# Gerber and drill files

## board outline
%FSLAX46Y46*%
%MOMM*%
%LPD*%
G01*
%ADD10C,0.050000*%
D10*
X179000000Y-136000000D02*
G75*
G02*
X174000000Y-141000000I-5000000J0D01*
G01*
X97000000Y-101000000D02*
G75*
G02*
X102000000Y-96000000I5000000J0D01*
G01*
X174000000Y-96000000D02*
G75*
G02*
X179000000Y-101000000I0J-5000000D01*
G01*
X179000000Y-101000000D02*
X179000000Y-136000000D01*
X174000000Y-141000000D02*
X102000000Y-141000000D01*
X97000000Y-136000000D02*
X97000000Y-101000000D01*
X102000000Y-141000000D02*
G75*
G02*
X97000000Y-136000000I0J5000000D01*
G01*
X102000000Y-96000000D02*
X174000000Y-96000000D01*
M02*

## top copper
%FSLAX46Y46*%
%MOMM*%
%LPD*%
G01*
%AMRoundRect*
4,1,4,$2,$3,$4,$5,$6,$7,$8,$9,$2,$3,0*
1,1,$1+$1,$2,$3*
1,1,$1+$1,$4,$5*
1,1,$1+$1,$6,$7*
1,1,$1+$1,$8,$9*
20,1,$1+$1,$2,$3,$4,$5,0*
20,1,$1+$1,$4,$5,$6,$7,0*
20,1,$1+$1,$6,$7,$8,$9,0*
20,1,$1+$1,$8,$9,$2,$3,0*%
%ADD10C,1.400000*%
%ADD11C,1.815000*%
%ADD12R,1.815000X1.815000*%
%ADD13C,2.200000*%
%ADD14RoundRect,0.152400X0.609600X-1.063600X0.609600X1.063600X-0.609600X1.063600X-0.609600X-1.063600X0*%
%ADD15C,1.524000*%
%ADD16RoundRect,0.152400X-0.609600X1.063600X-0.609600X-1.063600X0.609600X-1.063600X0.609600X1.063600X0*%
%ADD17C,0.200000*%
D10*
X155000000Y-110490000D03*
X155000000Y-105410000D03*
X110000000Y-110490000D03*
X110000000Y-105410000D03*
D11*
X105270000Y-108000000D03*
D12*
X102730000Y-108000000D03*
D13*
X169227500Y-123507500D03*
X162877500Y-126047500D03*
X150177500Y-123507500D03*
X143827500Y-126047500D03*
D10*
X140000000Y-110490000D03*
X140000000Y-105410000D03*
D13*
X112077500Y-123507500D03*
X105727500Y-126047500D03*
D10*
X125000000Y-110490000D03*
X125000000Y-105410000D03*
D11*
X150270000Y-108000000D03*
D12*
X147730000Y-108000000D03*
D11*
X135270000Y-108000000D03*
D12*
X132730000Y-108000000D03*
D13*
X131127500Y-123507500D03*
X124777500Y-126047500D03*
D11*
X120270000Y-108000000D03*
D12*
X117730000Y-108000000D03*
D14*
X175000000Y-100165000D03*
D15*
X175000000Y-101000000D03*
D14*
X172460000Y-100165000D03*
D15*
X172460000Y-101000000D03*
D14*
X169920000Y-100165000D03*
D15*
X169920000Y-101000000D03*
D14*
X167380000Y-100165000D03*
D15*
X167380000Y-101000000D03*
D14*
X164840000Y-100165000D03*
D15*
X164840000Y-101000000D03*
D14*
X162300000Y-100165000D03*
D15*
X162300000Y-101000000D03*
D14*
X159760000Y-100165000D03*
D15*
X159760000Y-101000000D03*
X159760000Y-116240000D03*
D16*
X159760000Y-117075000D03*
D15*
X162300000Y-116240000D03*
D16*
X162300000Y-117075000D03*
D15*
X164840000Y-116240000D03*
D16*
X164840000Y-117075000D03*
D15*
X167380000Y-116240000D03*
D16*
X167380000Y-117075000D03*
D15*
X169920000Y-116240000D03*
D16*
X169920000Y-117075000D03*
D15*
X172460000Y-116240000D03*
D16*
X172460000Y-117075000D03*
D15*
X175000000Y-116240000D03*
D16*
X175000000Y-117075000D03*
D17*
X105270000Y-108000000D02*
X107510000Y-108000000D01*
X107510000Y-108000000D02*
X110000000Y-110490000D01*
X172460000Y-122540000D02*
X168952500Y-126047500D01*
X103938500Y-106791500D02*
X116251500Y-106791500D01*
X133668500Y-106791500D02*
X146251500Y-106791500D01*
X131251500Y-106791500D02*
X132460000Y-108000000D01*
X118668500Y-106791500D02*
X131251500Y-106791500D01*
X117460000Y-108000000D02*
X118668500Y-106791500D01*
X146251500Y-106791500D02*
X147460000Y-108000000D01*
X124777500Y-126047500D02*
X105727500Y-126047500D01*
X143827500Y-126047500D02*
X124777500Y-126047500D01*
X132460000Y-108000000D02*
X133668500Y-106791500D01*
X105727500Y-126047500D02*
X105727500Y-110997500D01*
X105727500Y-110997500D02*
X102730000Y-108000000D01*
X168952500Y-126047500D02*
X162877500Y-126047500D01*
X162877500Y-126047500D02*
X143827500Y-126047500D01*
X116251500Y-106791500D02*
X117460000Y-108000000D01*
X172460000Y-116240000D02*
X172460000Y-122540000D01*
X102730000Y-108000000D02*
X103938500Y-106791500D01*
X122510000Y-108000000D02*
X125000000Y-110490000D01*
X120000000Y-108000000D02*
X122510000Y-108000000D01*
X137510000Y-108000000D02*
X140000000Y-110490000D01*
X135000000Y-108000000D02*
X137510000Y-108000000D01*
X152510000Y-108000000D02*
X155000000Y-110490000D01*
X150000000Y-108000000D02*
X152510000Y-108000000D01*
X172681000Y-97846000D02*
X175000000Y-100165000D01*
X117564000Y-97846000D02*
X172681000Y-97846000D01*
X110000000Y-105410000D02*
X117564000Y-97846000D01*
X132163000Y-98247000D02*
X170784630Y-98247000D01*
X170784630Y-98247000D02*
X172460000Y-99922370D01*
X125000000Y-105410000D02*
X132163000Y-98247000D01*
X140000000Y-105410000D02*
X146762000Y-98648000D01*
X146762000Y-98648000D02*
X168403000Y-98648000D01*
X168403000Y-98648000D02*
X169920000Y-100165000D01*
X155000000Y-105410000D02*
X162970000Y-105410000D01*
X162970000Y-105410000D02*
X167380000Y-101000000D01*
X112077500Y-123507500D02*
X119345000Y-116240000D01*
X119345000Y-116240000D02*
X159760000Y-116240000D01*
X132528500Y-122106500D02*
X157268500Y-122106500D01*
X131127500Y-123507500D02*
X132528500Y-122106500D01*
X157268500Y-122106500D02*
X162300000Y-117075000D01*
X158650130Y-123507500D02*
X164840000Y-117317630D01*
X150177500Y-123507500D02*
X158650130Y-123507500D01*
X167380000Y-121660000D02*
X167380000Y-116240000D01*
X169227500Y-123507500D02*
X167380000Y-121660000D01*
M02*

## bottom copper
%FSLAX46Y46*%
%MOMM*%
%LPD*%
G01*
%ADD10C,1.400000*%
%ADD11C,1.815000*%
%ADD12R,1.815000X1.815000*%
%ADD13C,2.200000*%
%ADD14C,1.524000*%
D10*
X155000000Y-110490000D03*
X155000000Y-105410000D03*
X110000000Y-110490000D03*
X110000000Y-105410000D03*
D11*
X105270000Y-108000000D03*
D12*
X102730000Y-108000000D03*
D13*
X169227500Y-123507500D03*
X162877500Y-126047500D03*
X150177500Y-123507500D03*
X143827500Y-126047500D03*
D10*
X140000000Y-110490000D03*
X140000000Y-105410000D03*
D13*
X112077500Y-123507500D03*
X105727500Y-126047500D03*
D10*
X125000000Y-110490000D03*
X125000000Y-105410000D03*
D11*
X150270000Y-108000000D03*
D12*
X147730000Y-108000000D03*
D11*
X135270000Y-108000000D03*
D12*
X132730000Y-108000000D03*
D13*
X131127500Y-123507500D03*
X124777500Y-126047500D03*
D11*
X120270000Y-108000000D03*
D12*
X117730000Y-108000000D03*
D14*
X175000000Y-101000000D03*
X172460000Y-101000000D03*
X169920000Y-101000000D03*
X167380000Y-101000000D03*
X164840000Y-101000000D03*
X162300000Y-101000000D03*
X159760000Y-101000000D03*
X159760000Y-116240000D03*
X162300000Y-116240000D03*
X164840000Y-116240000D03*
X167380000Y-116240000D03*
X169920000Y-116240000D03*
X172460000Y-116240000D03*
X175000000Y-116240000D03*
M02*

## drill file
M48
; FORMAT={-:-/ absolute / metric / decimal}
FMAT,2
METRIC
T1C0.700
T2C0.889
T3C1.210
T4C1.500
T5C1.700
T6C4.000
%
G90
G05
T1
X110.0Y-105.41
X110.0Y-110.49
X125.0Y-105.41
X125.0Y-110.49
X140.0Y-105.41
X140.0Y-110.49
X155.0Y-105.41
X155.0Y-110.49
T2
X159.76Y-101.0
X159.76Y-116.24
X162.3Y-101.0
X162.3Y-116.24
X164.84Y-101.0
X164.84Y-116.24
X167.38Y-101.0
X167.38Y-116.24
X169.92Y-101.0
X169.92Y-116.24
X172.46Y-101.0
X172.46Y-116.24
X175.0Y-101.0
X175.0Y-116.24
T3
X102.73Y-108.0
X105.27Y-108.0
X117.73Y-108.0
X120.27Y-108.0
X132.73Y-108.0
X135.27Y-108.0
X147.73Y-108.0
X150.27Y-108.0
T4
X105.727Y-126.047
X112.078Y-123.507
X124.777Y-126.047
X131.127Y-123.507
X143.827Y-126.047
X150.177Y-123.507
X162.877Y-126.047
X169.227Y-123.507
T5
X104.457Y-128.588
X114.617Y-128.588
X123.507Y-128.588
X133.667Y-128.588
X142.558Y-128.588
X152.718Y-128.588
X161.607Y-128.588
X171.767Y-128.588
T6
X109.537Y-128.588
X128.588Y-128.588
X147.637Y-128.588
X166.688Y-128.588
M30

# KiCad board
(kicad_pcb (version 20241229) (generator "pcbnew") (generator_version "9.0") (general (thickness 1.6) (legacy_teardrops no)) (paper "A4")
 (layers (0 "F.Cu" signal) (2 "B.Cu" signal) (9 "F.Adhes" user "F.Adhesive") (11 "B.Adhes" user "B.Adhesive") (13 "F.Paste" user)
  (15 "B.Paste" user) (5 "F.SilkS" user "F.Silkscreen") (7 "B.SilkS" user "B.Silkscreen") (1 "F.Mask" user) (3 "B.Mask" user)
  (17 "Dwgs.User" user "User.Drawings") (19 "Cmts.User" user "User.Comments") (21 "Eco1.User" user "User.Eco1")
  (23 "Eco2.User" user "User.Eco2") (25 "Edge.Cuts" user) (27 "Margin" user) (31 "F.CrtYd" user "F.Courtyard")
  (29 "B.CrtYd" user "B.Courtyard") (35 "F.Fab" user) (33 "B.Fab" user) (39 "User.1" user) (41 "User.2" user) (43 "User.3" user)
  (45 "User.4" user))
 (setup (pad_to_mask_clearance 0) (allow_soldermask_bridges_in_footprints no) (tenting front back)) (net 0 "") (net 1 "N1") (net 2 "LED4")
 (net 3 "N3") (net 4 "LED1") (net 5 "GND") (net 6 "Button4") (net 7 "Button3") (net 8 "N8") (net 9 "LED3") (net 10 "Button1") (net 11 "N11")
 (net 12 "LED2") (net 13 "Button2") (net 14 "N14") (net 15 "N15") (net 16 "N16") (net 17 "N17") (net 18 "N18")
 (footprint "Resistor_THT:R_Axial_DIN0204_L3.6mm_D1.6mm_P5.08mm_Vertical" (layer "F.Cu") (at 155 110.49 90)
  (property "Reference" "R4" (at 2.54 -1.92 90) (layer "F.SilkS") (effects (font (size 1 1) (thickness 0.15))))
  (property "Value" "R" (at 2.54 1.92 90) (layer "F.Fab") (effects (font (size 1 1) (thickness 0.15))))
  (pad "1" thru_hole circle (at 0 0 90) (size 1.4 1.4) (drill 0.7) (layers "*.Cu" "*.Mask") (remove_unused_layers no) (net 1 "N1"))
  (pad "2" thru_hole circle (at 5.08 0 90) (size 1.4 1.4) (drill 0.7) (layers "*.Cu" "*.Mask") (remove_unused_layers no) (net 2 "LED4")))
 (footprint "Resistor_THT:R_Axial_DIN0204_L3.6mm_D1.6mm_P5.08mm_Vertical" (layer "F.Cu") (at 110 110.49 90)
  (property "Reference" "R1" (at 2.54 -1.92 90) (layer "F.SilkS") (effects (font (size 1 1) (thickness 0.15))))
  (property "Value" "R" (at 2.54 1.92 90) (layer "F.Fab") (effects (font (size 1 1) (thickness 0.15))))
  (pad "1" thru_hole circle (at 0 0 90) (size 1.4 1.4) (drill 0.7) (layers "*.Cu" "*.Mask") (remove_unused_layers no) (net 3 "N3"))
  (pad "2" thru_hole circle (at 5.08 0 90) (size 1.4 1.4) (drill 0.7) (layers "*.Cu" "*.Mask") (remove_unused_layers no) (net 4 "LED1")))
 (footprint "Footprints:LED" (layer "F.Cu") (at 104 108)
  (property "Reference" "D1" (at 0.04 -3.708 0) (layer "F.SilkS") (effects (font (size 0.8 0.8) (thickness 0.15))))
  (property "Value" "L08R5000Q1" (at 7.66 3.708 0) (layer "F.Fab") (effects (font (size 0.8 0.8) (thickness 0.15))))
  (pad "A" thru_hole circle (at 1.27 0) (size 1.815 1.815) (drill 1.21) (layers "*.Cu" "*.Mask") (remove_unused_layers no) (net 3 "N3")
   (solder_mask_margin 0.102))
  (pad "C" thru_hole rect (at -1.27 0) (size 1.815 1.815) (drill 1.21) (layers "*.Cu" "*.Mask") (remove_unused_layers no) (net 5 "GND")
   (solder_mask_margin 0.102)))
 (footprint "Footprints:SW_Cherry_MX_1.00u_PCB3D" (layer "F.Cu") (at 169.2275 123.5075)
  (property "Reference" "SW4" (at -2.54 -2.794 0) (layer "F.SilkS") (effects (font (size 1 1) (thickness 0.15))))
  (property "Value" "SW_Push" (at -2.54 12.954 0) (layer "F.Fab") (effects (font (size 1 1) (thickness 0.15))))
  (pad "" np_thru_hole circle (at -7.62 5.08) (size 1.7 1.7) (drill 1.7) (layers "*.Cu" "*.Mask"))
  (pad "" np_thru_hole circle (at -2.54 5.08) (size 4 4) (drill 4) (layers "*.Cu" "*.Mask"))
  (pad "" np_thru_hole circle (at 2.54 5.08) (size 1.7 1.7) (drill 1.7) (layers "*.Cu" "*.Mask"))
  (pad "1" thru_hole circle (at 0 0) (size 2.2 2.2) (drill 1.5) (layers "*.Cu" "*.Mask") (remove_unused_layers no) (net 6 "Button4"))
  (pad "2" thru_hole circle (at -6.35 2.54) (size 2.2 2.2) (drill 1.5) (layers "*.Cu" "*.Mask") (remove_unused_layers no) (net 5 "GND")))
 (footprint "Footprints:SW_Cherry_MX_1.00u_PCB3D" (layer "F.Cu") (at 150.1775 123.5075)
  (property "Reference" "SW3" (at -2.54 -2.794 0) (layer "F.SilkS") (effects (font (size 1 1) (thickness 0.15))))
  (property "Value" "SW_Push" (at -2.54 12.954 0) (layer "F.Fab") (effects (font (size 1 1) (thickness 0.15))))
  (pad "" np_thru_hole circle (at -7.62 5.08) (size 1.7 1.7) (drill 1.7) (layers "*.Cu" "*.Mask"))
  (pad "" np_thru_hole circle (at -2.54 5.08) (size 4 4) (drill 4) (layers "*.Cu" "*.Mask"))
  (pad "" np_thru_hole circle (at 2.54 5.08) (size 1.7 1.7) (drill 1.7) (layers "*.Cu" "*.Mask"))
  (pad "1" thru_hole circle (at 0 0) (size 2.2 2.2) (drill 1.5) (layers "*.Cu" "*.Mask") (remove_unused_layers no) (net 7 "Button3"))
  (pad "2" thru_hole circle (at -6.35 2.54) (size 2.2 2.2) (drill 1.5) (layers "*.Cu" "*.Mask") (remove_unused_layers no) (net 5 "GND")))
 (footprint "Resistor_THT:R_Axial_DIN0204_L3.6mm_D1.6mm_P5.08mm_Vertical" (layer "F.Cu") (at 140 110.49 90)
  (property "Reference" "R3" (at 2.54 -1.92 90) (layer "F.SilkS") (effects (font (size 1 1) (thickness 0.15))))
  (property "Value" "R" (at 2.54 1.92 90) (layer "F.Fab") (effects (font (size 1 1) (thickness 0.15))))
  (pad "1" thru_hole circle (at 0 0 90) (size 1.4 1.4) (drill 0.7) (layers "*.Cu" "*.Mask") (remove_unused_layers no) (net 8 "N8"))
  (pad "2" thru_hole circle (at 5.08 0 90) (size 1.4 1.4) (drill 0.7) (layers "*.Cu" "*.Mask") (remove_unused_layers no) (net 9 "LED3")))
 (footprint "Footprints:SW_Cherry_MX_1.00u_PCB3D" (layer "F.Cu") (at 112.0775 123.5075)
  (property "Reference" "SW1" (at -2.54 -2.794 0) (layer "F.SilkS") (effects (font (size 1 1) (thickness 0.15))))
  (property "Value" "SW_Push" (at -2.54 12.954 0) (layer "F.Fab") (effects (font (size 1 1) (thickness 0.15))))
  (pad "" np_thru_hole circle (at -7.62 5.08) (size 1.7 1.7) (drill 1.7) (layers "*.Cu" "*.Mask"))
  (pad "" np_thru_hole circle (at -2.54 5.08) (size 4 4) (drill 4) (layers "*.Cu" "*.Mask"))
  (pad "" np_thru_hole circle (at 2.54 5.08) (size 1.7 1.7) (drill 1.7) (layers "*.Cu" "*.Mask"))
  (pad "1" thru_hole circle (at 0 0) (size 2.2 2.2) (drill 1.5) (layers "*.Cu" "*.Mask") (remove_unused_layers no) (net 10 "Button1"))
  (pad "2" thru_hole circle (at -6.35 2.54) (size 2.2 2.2) (drill 1.5) (layers "*.Cu" "*.Mask") (remove_unused_layers no) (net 5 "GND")))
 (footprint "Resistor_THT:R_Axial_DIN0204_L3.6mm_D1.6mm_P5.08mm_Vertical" (layer "F.Cu") (at 125 110.49 90)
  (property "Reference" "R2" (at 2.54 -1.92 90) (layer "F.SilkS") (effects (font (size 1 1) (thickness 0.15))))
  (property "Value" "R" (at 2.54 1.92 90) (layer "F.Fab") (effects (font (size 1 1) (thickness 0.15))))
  (pad "1" thru_hole circle (at 0 0 90) (size 1.4 1.4) (drill 0.7) (layers "*.Cu" "*.Mask") (remove_unused_layers no) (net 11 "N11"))
  (pad "2" thru_hole circle (at 5.08 0 90) (size 1.4 1.4) (drill 0.7) (layers "*.Cu" "*.Mask") (remove_unused_layers no) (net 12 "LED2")))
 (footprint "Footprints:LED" (layer "F.Cu") (at 149 108)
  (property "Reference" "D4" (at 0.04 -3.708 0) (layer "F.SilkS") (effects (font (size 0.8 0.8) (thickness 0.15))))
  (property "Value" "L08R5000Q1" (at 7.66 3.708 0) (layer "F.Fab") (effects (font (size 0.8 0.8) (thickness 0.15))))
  (pad "A" thru_hole circle (at 1.27 0) (size 1.815 1.815) (drill 1.21) (layers "*.Cu" "*.Mask") (remove_unused_layers no) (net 1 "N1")
   (solder_mask_margin 0.102))
  (pad "C" thru_hole rect (at -1.27 0) (size 1.815 1.815) (drill 1.21) (layers "*.Cu" "*.Mask") (remove_unused_layers no) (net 5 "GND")
   (solder_mask_margin 0.102)))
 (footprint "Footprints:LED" (layer "F.Cu") (at 134 108)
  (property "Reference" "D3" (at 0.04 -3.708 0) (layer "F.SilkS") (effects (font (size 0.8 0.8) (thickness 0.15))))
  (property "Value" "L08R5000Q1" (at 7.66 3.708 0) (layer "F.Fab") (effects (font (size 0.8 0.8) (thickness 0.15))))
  (pad "A" thru_hole circle (at 1.27 0) (size 1.815 1.815) (drill 1.21) (layers "*.Cu" "*.Mask") (remove_unused_layers no) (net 8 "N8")
   (solder_mask_margin 0.102))
  (pad "C" thru_hole rect (at -1.27 0) (size 1.815 1.815) (drill 1.21) (layers "*.Cu" "*.Mask") (remove_unused_layers no) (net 5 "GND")
   (solder_mask_margin 0.102)))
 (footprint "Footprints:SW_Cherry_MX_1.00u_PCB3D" (layer "F.Cu") (at 131.1275 123.5075)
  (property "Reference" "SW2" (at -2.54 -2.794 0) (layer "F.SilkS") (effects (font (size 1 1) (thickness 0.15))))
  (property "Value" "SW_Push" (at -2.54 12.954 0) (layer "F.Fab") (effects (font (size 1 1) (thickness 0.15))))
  (pad "" np_thru_hole circle (at -7.62 5.08) (size 1.7 1.7) (drill 1.7) (layers "*.Cu" "*.Mask"))
  (pad "" np_thru_hole circle (at -2.54 5.08) (size 4 4) (drill 4) (layers "*.Cu" "*.Mask"))
  (pad "" np_thru_hole circle (at 2.54 5.08) (size 1.7 1.7) (drill 1.7) (layers "*.Cu" "*.Mask"))
  (pad "1" thru_hole circle (at 0 0) (size 2.2 2.2) (drill 1.5) (layers "*.Cu" "*.Mask") (remove_unused_layers no) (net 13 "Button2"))
  (pad "2" thru_hole circle (at -6.35 2.54) (size 2.2 2.2) (drill 1.5) (layers "*.Cu" "*.Mask") (remove_unused_layers no) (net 5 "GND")))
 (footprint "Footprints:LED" (layer "F.Cu") (at 119 108)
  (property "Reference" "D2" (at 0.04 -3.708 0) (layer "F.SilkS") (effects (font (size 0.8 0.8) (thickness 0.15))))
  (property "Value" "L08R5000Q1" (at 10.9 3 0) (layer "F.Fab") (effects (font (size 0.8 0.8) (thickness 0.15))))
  (pad "A" thru_hole circle (at 1.27 0) (size 1.815 1.815) (drill 1.21) (layers "*.Cu" "*.Mask") (remove_unused_layers no) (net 11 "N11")
   (solder_mask_margin 0.102))
  (pad "C" thru_hole rect (at -1.27 0) (size 1.815 1.815) (drill 1.21) (layers "*.Cu" "*.Mask") (remove_unused_layers no) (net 5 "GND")
   (solder_mask_margin 0.102)))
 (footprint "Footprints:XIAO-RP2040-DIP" (layer "F.Cu") (at 167.38 108.62 -90)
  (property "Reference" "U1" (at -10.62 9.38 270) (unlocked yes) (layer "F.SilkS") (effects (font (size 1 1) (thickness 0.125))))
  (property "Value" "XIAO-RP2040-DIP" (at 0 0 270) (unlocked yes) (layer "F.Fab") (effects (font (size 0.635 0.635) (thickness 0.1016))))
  (pad "1" smd roundrect (at -8.455 -7.62 90) (size 2.432 1.524) (layers "F.Cu" "F.Mask") (roundrect_rratio 0.1) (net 4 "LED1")
   (thermal_bridge_angle 45))
  (pad "1" thru_hole circle (at -7.62 -7.62 90) (size 1.524 1.524) (drill 0.889) (layers "*.Cu" "*.Mask") (remove_unused_layers no)
   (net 4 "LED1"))
  (pad "2" smd roundrect (at -8.455 -5.08 90) (size 2.432 1.524) (layers "F.Cu" "F.Mask") (roundrect_rratio 0.1) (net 12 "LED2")
   (thermal_bridge_angle 45))
  (pad "2" thru_hole circle (at -7.62 -5.08 90) (size 1.524 1.524) (drill 0.889) (layers "*.Cu" "*.Mask") (remove_unused_layers no)
   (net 12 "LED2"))
  (pad "3" smd roundrect (at -8.455 -2.54 90) (size 2.432 1.524) (layers "F.Cu" "F.Mask") (roundrect_rratio 0.1) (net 9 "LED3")
   (thermal_bridge_angle 45))
  (pad "3" thru_hole circle (at -7.62 -2.54 90) (size 1.524 1.524) (drill 0.889) (layers "*.Cu" "*.Mask") (remove_unused_layers no)
   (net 9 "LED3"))
  (pad "4" smd roundrect (at -8.455 0 90) (size 2.432 1.524) (layers "F.Cu" "F.Mask") (roundrect_rratio 0.1) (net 2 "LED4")
   (thermal_bridge_angle 45))
  (pad "4" thru_hole circle (at -7.62 0 90) (size 1.524 1.524) (drill 0.889) (layers "*.Cu" "*.Mask") (remove_unused_layers no)
   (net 2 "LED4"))
  (pad "5" smd roundrect (at -8.455 2.54 90) (size 2.432 1.524) (layers "F.Cu" "F.Mask") (roundrect_rratio 0.1) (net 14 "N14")
   (thermal_bridge_angle 45))
  (pad "5" thru_hole circle (at -7.62 2.54 90) (size 1.524 1.524) (drill 0.889) (layers "*.Cu" "*.Mask") (remove_unused_layers no)
   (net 14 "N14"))
  (pad "6" smd roundrect (at -8.455 5.08 90) (size 2.432 1.524) (layers "F.Cu" "F.Mask") (roundrect_rratio 0.1) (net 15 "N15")
   (thermal_bridge_angle 45))
  (pad "6" thru_hole circle (at -7.62 5.08 90) (size 1.524 1.524) (drill 0.889) (layers "*.Cu" "*.Mask") (remove_unused_layers no)
   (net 15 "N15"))
  (pad "7" smd roundrect (at -8.455 7.62 90) (size 2.432 1.524) (layers "F.Cu" "F.Mask") (roundrect_rratio 0.1) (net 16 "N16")
   (thermal_bridge_angle 45))
  (pad "7" thru_hole circle (at -7.62 7.62 90) (size 1.524 1.524) (drill 0.889) (layers "*.Cu" "*.Mask") (remove_unused_layers no)
   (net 16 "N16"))
  (pad "8" thru_hole circle (at 7.62 7.62 270) (size 1.524 1.524) (drill 0.889) (layers "*.Cu" "*.Mask") (remove_unused_layers no)
   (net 10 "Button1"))
  (pad "8" smd roundrect (at 8.455 7.62 270) (size 2.432 1.524) (layers "F.Cu" "F.Mask") (roundrect_rratio 0.1) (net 10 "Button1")
   (thermal_bridge_angle 45))
  (pad "9" thru_hole circle (at 7.62 5.08 270) (size 1.524 1.524) (drill 0.889) (layers "*.Cu" "*.Mask") (remove_unused_layers no)
   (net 13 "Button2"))
  (pad "9" smd roundrect (at 8.455 5.08 270) (size 2.432 1.524) (layers "F.Cu" "F.Mask") (roundrect_rratio 0.1) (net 13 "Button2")
   (thermal_bridge_angle 45))
  (pad "10" thru_hole circle (at 7.62 2.54 270) (size 1.524 1.524) (drill 0.889) (layers "*.Cu" "*.Mask") (remove_unused_layers no)
   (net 7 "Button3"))
  (pad "10" smd roundrect (at 8.455 2.54 270) (size 2.432 1.524) (layers "F.Cu" "F.Mask") (roundrect_rratio 0.1) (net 7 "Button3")
   (thermal_bridge_angle 45))
  (pad "11" thru_hole circle (at 7.62 0 270) (size 1.524 1.524) (drill 0.889) (layers "*.Cu" "*.Mask") (remove_unused_layers no)
   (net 6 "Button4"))
  (pad "11" smd roundrect (at 8.455 0 270) (size 2.432 1.524) (layers "F.Cu" "F.Mask") (roundrect_rratio 0.1) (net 6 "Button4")
   (thermal_bridge_angle 45))
  (pad "12" thru_hole circle (at 7.62 -2.54 270) (size 1.524 1.524) (drill 0.889) (layers "*.Cu" "*.Mask") (remove_unused_layers no)
   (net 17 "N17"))
  (pad "12" smd roundrect (at 8.455 -2.54 270) (size 2.432 1.524) (layers "F.Cu" "F.Mask") (roundrect_rratio 0.1) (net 17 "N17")
   (thermal_bridge_angle 45))
  (pad "13" thru_hole circle (at 7.62 -5.08 270) (size 1.524 1.524) (drill 0.889) (layers "*.Cu" "*.Mask") (remove_unused_layers no)
   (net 5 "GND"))
  (pad "13" smd roundrect (at 8.455 -5.08 270) (size 2.432 1.524) (layers "F.Cu" "F.Mask") (roundrect_rratio 0.1) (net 5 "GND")
   (thermal_bridge_angle 45))
  (pad "14" thru_hole circle (at 7.62 -7.62 270) (size 1.524 1.524) (drill 0.889) (layers "*.Cu" "*.Mask") (remove_unused_layers no)
   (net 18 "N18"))
  (pad "14" smd roundrect (at 8.455 -7.62 270) (size 2.432 1.524) (layers "F.Cu" "F.Mask") (roundrect_rratio 0.1) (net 18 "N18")
   (thermal_bridge_angle 45)))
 (gr_arc (start 179 136) (mid 177.535534 139.535534) (end 174 141) (stroke (width 0.05) (type default)) (layer "Edge.Cuts"))
 (gr_arc (start 97 101) (mid 98.464466 97.464466) (end 102 96) (stroke (width 0.05) (type default)) (layer "Edge.Cuts"))
 (gr_arc (start 174 96) (mid 177.535534 97.464466) (end 179 101) (stroke (width 0.05) (type default)) (layer "Edge.Cuts"))
 (gr_line (start 179 101) (end 179 136) (stroke (width 0.05) (type default)) (layer "Edge.Cuts"))
 (gr_line (start 174 141) (end 102 141) (stroke (width 0.05) (type default)) (layer "Edge.Cuts"))
 (gr_line (start 97 136) (end 97 101) (stroke (width 0.05) (type default)) (layer "Edge.Cuts"))
 (gr_arc (start 102 141) (mid 98.464466 139.535534) (end 97 136) (stroke (width 0.05) (type default)) (layer "Edge.Cuts"))
 (gr_line (start 102 96) (end 174 96) (stroke (width 0.05) (type default)) (layer "Edge.Cuts"))
 (segment (start 105.27 108) (end 107.51 108) (width 0.2) (layer "F.Cu") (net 3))
 (segment (start 107.51 108) (end 110 110.49) (width 0.2) (layer "F.Cu") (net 3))
 (segment (start 172.46 122.54) (end 168.9525 126.0475) (width 0.2) (layer "F.Cu") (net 5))
 (segment (start 103.9385 106.7915) (end 116.2515 106.7915) (width 0.2) (layer "F.Cu") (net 5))
 (segment (start 133.6685 106.7915) (end 146.2515 106.7915) (width 0.2) (layer "F.Cu") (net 5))
 (segment (start 131.2515 106.7915) (end 132.46 108) (width 0.2) (layer "F.Cu") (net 5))
 (segment (start 118.6685 106.7915) (end 131.2515 106.7915) (width 0.2) (layer "F.Cu") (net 5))
 (segment (start 117.46 108) (end 118.6685 106.7915) (width 0.2) (layer "F.Cu") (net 5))
 (segment (start 146.2515 106.7915) (end 147.46 108) (width 0.2) (layer "F.Cu") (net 5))
 (segment (start 124.7775 126.0475) (end 105.7275 126.0475) (width 0.2) (layer "F.Cu") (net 5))
 (segment (start 143.8275 126.0475) (end 124.7775 126.0475) (width 0.2) (layer "F.Cu") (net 5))
 (segment (start 132.46 108) (end 133.6685 106.7915) (width 0.2) (layer "F.Cu") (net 5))
 (segment (start 105.7275 126.0475) (end 105.7275 110.9975) (width 0.2) (layer "F.Cu") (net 5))
 (segment (start 105.7275 110.9975) (end 102.73 108) (width 0.2) (layer "F.Cu") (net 5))
 (segment (start 168.9525 126.0475) (end 162.8775 126.0475) (width 0.2) (layer "F.Cu") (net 5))
 (segment (start 162.8775 126.0475) (end 143.8275 126.0475) (width 0.2) (layer "F.Cu") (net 5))
 (segment (start 116.2515 106.7915) (end 117.46 108) (width 0.2) (layer "F.Cu") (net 5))
 (segment (start 172.46 116.24) (end 172.46 122.54) (width 0.2) (layer "F.Cu") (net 5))
 (segment (start 102.73 108) (end 103.9385 106.7915) (width 0.2) (layer "F.Cu") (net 5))
 (segment (start 122.51 108) (end 125 110.49) (width 0.2) (layer "F.Cu") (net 11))
 (segment (start 120 108) (end 122.51 108) (width 0.2) (layer "F.Cu") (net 11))
 (segment (start 137.51 108) (end 140 110.49) (width 0.2) (layer "F.Cu") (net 8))
 (segment (start 135 108) (end 137.51 108) (width 0.2) (layer "F.Cu") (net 8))
 (segment (start 152.51 108) (end 155 110.49) (width 0.2) (layer "F.Cu") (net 1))
 (segment (start 150 108) (end 152.51 108) (width 0.2) (layer "F.Cu") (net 1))
 (segment (start 172.681 97.846) (end 175 100.165) (width 0.2) (layer "F.Cu") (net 4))
 (segment (start 117.564 97.846) (end 172.681 97.846) (width 0.2) (layer "F.Cu") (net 4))
 (segment (start 110 105.41) (end 117.564 97.846) (width 0.2) (layer "F.Cu") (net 4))
 (segment (start 132.163 98.247) (end 170.78463 98.247) (width 0.2) (layer "F.Cu") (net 12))
 (segment (start 170.78463 98.247) (end 172.46 99.92237) (width 0.2) (layer "F.Cu") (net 12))
 (segment (start 125 105.41) (end 132.163 98.247) (width 0.2) (layer "F.Cu") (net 12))
 (segment (start 140 105.41) (end 146.762 98.648) (width 0.2) (layer "F.Cu") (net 9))
 (segment (start 146.762 98.648) (end 168.403 98.648) (width 0.2) (layer "F.Cu") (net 9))
 (segment (start 168.403 98.648) (end 169.92 100.165) (width 0.2) (layer "F.Cu") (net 9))
 (segment (start 155 105.41) (end 162.97 105.41) (width 0.2) (layer "F.Cu") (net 2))
 (segment (start 162.97 105.41) (end 167.38 101) (width 0.2) (layer "F.Cu") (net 2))
 (segment (start 112.0775 123.5075) (end 119.345 116.24) (width 0.2) (layer "F.Cu") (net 10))
 (segment (start 119.345 116.24) (end 159.76 116.24) (width 0.2) (layer "F.Cu") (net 10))
 (segment (start 132.5285 122.1065) (end 157.2685 122.1065) (width 0.2) (layer "F.Cu") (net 13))
 (segment (start 131.1275 123.5075) (end 132.5285 122.1065) (width 0.2) (layer "F.Cu") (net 13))
 (segment (start 157.2685 122.1065) (end 162.3 117.075) (width 0.2) (layer "F.Cu") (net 13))
 (segment (start 158.65013 123.5075) (end 164.84 117.31763) (width 0.2) (layer "F.Cu") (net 7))
 (segment (start 150.1775 123.5075) (end 158.65013 123.5075) (width 0.2) (layer "F.Cu") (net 7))
 (segment (start 167.38 121.66) (end 167.38 116.24) (width 0.2) (layer "F.Cu") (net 6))
 (segment (start 169.2275 123.5075) (end 167.38 121.66) (width 0.2) (layer "F.Cu") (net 6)))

